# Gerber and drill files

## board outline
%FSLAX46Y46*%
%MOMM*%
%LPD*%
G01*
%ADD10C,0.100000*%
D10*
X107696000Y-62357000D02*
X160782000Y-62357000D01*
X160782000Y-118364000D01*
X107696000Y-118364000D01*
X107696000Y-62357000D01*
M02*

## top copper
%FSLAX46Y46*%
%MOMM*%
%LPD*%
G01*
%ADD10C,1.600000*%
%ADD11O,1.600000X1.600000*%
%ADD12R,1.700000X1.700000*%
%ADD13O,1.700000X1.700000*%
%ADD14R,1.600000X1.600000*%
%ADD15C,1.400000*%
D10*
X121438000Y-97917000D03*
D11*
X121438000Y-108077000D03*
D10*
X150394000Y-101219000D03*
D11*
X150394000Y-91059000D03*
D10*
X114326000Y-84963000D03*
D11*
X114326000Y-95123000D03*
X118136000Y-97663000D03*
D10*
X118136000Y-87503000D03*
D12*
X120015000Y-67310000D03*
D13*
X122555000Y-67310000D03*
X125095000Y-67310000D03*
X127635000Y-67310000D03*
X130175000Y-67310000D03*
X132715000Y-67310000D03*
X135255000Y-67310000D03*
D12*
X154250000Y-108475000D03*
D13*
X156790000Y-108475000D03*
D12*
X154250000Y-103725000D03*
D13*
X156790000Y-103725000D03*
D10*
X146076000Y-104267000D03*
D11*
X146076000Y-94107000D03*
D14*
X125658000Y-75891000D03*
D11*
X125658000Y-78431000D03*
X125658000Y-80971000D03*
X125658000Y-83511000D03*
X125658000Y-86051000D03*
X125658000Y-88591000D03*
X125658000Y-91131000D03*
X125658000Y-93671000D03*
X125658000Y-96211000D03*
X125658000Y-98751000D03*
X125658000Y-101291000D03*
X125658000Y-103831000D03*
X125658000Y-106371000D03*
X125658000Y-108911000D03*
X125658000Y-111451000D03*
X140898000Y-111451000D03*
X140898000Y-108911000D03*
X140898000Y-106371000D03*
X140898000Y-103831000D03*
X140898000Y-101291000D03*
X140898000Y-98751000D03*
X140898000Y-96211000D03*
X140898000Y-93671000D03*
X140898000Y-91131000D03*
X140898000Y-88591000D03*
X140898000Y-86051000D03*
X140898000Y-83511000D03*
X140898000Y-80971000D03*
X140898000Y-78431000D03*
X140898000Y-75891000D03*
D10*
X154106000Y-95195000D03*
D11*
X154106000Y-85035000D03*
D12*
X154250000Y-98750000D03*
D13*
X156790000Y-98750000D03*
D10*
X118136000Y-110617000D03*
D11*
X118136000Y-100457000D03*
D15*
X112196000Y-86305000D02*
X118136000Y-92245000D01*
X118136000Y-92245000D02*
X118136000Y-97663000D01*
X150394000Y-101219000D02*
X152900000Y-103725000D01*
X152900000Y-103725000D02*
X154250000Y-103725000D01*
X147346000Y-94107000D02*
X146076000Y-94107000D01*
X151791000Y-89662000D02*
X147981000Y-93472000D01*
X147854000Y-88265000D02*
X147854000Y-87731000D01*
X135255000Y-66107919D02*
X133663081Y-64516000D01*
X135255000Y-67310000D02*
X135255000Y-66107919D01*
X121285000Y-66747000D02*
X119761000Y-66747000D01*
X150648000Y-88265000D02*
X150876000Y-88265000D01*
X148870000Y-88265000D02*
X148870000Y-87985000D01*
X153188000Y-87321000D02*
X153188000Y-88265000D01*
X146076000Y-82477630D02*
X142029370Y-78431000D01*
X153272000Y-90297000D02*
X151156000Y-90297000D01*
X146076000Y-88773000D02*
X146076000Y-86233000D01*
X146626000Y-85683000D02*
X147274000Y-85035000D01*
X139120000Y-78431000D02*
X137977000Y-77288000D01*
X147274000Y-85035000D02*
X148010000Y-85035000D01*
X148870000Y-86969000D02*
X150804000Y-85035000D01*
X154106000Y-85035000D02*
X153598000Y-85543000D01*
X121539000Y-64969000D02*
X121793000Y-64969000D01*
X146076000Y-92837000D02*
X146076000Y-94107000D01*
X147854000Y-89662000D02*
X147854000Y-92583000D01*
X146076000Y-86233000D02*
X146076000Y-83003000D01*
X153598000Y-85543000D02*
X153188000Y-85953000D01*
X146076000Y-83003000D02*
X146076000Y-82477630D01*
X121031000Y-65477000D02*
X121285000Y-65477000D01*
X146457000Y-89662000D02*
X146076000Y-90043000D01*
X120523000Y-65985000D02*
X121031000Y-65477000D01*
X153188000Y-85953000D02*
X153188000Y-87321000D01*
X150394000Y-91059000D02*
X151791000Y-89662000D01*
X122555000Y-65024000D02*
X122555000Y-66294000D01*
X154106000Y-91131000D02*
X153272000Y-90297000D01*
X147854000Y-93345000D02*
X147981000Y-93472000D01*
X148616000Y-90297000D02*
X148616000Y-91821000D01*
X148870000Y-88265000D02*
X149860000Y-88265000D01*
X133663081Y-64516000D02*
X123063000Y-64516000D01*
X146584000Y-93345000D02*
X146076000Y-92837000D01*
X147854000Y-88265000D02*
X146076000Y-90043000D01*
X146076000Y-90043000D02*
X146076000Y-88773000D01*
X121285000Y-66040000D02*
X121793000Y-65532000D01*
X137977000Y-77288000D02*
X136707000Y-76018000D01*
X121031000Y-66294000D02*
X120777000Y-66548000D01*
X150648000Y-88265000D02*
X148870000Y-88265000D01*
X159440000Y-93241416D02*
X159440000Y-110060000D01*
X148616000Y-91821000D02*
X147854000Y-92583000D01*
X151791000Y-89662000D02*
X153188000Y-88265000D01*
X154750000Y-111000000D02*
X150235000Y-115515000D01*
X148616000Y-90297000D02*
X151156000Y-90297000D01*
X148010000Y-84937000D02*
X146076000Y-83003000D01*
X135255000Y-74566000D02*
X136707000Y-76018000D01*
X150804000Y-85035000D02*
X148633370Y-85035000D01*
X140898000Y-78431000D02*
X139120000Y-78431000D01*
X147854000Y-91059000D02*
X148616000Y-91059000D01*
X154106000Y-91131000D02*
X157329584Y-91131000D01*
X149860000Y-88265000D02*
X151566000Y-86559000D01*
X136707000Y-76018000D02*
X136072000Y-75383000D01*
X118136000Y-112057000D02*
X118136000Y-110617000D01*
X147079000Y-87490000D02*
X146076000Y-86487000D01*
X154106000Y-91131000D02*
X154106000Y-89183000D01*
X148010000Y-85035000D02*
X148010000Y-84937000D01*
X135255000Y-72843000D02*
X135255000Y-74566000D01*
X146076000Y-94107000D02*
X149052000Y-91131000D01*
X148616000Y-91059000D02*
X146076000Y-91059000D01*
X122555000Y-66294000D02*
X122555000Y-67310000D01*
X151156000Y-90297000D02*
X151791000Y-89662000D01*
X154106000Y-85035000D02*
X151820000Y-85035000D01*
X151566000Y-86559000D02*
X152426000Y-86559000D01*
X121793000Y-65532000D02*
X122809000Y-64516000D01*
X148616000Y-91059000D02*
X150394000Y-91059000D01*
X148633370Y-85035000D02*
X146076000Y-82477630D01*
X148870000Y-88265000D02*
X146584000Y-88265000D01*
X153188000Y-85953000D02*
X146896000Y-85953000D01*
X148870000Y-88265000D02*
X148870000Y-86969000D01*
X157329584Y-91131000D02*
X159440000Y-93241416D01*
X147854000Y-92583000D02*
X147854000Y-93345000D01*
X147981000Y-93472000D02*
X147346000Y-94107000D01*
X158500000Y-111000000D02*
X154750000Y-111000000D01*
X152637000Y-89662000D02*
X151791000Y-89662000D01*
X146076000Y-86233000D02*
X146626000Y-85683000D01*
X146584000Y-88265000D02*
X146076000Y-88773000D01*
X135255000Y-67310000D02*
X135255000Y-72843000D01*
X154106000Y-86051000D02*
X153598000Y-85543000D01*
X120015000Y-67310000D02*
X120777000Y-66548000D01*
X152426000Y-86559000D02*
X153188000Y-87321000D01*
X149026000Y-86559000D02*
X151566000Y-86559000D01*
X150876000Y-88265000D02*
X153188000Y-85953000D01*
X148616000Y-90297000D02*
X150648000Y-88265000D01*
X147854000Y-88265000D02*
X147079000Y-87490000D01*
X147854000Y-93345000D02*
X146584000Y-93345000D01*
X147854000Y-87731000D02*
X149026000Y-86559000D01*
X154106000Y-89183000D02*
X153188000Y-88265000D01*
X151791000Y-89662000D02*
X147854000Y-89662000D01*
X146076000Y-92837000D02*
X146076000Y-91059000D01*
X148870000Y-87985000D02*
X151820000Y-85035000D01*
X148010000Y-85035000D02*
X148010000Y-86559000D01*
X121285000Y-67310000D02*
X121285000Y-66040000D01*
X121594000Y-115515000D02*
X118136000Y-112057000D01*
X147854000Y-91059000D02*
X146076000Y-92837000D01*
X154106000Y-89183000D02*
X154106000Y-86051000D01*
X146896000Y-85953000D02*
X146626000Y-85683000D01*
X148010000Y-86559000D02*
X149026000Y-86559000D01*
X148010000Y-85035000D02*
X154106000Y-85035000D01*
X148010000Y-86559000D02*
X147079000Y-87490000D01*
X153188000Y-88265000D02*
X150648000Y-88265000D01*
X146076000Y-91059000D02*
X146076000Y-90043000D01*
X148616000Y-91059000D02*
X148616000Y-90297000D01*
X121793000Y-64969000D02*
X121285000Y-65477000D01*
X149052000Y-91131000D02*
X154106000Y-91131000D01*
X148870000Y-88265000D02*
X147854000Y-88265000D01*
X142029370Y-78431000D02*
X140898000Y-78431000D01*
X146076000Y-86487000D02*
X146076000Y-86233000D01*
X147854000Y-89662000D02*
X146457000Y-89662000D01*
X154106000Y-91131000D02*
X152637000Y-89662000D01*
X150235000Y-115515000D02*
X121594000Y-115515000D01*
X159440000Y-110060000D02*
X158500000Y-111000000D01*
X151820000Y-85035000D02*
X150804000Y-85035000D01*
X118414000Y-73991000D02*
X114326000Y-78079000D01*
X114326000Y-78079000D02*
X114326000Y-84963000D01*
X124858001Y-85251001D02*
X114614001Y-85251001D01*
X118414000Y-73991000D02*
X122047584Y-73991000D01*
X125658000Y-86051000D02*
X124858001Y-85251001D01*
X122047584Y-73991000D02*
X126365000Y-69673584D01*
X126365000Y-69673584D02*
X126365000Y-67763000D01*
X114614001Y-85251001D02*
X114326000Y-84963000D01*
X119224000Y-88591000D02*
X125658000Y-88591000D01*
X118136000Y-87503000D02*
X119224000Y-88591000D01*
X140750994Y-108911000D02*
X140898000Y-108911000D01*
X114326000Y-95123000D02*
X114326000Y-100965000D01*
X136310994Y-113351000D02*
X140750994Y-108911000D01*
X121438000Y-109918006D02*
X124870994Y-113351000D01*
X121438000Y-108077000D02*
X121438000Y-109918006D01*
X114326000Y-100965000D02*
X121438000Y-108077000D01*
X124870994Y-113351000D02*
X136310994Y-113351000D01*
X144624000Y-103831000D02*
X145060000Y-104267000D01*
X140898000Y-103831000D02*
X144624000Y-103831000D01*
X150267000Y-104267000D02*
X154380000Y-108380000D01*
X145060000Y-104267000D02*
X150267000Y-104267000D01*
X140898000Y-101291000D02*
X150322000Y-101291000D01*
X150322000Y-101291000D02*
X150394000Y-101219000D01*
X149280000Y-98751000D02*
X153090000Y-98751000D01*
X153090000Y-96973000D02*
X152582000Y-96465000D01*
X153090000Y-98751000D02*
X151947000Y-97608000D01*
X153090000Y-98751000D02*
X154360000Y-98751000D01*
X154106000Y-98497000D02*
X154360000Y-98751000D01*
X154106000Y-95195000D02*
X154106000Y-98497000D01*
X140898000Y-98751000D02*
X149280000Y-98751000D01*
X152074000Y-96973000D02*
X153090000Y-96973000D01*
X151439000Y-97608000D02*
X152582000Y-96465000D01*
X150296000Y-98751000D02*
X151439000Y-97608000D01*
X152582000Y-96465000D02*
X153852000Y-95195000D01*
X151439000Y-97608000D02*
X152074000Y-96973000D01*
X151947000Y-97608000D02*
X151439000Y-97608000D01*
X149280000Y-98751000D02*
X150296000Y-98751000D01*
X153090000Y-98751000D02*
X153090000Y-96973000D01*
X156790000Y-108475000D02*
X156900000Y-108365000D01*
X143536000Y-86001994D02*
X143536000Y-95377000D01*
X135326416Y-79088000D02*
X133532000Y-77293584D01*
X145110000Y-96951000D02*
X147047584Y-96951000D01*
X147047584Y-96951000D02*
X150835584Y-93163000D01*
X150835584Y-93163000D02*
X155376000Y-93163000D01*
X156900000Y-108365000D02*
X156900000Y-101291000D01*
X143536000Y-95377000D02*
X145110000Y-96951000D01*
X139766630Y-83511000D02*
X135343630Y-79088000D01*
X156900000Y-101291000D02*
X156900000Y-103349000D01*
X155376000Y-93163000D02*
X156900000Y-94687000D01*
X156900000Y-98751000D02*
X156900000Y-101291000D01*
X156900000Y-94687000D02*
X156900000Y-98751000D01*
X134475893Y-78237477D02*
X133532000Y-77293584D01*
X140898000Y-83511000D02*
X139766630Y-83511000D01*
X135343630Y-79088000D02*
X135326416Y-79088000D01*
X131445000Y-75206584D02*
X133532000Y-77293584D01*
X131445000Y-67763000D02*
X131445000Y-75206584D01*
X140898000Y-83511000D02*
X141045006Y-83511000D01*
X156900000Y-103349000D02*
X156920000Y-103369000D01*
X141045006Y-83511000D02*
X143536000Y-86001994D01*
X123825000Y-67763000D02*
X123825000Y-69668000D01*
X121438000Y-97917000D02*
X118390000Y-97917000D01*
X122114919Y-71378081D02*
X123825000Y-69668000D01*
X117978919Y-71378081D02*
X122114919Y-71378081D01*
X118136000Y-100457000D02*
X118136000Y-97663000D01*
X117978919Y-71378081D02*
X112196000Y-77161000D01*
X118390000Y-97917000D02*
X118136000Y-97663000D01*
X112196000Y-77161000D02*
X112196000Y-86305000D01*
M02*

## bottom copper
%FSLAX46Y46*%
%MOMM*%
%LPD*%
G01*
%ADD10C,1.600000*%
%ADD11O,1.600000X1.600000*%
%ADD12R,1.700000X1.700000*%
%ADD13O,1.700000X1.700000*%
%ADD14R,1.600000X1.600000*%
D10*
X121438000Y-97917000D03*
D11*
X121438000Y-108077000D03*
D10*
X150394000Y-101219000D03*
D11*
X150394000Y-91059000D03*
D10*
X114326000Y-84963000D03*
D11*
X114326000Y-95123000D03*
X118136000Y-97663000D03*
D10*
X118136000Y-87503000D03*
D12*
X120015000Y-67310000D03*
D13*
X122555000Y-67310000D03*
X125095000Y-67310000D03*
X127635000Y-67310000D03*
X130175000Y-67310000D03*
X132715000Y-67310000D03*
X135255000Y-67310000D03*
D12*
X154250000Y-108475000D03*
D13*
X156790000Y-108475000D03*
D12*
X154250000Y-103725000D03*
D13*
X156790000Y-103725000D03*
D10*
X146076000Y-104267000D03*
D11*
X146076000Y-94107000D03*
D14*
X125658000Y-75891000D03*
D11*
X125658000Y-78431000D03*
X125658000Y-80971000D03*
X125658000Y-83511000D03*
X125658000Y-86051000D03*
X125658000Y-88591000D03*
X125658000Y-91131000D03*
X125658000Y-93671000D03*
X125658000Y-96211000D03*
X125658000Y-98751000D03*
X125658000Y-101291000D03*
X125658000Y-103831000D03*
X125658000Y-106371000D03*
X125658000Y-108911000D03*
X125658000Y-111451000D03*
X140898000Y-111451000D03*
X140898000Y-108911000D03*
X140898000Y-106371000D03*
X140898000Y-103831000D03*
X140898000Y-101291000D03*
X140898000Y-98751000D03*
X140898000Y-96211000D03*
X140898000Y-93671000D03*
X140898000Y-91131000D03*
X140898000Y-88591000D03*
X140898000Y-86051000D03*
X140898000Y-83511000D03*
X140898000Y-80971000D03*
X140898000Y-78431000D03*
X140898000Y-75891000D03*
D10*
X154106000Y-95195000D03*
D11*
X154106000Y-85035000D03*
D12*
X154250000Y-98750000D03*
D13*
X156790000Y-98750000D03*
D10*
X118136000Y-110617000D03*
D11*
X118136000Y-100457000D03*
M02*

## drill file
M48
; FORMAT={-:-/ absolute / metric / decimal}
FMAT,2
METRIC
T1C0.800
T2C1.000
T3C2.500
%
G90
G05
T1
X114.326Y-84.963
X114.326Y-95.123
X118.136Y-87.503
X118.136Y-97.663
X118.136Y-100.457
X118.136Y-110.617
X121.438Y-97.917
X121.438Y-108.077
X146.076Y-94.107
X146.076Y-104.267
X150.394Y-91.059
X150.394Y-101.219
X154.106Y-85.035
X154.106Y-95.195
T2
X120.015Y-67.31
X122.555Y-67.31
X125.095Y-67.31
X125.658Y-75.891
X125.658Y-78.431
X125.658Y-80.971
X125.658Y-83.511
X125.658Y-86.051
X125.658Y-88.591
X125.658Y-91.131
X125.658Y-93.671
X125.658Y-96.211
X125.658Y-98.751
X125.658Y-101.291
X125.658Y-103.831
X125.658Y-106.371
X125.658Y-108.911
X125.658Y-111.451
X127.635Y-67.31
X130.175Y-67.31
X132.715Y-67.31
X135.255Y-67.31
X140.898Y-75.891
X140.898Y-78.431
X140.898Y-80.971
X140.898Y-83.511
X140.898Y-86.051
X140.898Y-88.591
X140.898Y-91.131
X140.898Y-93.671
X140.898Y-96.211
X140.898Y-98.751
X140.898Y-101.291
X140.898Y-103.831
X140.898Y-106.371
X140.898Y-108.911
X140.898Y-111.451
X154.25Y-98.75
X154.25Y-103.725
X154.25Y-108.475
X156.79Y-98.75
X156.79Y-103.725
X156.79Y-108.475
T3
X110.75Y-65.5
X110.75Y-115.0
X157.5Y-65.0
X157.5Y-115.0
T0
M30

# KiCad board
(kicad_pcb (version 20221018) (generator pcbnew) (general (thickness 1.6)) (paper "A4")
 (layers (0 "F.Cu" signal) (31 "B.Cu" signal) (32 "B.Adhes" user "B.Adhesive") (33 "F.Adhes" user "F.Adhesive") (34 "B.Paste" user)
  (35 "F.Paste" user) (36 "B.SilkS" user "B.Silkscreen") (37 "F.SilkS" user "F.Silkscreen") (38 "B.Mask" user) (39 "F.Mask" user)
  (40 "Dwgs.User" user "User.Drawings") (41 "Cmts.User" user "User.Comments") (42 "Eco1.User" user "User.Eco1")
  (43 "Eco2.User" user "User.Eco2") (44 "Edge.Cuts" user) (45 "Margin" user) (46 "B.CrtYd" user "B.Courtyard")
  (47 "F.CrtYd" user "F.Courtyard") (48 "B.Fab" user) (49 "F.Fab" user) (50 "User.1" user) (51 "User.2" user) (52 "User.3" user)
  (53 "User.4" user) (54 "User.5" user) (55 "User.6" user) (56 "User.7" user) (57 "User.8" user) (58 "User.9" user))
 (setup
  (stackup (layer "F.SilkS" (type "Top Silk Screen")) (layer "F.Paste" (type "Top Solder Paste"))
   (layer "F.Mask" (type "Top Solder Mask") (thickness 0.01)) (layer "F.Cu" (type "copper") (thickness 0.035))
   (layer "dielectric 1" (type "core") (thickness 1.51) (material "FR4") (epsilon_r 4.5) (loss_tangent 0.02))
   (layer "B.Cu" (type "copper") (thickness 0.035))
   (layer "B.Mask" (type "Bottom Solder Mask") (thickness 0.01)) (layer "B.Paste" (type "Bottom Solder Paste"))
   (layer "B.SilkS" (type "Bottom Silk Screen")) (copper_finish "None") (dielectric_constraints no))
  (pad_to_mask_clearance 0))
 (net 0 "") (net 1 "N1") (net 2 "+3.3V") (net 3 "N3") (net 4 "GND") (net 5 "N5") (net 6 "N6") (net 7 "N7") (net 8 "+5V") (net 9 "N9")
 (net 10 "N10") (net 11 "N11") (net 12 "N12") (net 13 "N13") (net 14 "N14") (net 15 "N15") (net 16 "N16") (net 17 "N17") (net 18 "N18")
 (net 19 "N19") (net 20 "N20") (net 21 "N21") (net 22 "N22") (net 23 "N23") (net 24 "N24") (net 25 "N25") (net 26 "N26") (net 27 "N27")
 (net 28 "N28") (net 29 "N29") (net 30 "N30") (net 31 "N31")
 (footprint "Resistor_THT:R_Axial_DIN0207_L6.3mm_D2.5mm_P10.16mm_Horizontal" (layer "F.Cu") (at 121.438 97.917 -90)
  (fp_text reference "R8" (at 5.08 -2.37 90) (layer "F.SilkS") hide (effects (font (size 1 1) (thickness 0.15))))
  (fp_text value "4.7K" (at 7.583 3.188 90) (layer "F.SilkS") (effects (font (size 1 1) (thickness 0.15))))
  (pad "1" thru_hole circle (at 0 0 270) (size 1.6 1.6) (drill 0.8) (layers "*.Cu" "*.Mask") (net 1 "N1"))
  (pad "2" thru_hole oval (at 10.16 0 270) (size 1.6 1.6) (drill 0.8) (layers "*.Cu" "*.Mask") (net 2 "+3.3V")))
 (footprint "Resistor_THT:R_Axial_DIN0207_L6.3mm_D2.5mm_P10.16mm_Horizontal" (layer "F.Cu") (at 150.394 101.219 90)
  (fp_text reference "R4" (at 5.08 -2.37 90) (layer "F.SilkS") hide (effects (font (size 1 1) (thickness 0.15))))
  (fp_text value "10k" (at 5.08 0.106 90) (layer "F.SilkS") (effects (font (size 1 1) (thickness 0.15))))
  (pad "1" thru_hole circle (at 0 0 90) (size 1.6 1.6) (drill 0.8) (layers "*.Cu" "*.Mask") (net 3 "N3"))
  (pad "2" thru_hole oval (at 10.16 0 90) (size 1.6 1.6) (drill 0.8) (layers "*.Cu" "*.Mask") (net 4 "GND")))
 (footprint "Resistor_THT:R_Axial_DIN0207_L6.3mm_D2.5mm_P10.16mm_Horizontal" (layer "F.Cu") (at 114.326 84.963 -90)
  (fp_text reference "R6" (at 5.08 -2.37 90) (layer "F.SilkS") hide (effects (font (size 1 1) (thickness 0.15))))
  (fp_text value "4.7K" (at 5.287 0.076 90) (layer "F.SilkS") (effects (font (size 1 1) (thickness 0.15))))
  (pad "1" thru_hole circle (at 0 0 270) (size 1.6 1.6) (drill 0.8) (layers "*.Cu" "*.Mask") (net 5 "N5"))
  (pad "2" thru_hole oval (at 10.16 0 270) (size 1.6 1.6) (drill 0.8) (layers "*.Cu" "*.Mask") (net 2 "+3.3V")))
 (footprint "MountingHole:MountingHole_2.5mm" (layer "F.Cu") (at 157.5 115)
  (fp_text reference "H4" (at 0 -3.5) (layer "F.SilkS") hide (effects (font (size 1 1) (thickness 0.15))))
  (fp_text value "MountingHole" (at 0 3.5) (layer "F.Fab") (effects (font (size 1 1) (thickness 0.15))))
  (pad "" np_thru_hole circle (at 0 0) (size 2.5 2.5) (drill 2.5) (layers "*.Cu" "*.Mask")))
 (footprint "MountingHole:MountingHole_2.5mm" (layer "F.Cu") (at 110.75 115)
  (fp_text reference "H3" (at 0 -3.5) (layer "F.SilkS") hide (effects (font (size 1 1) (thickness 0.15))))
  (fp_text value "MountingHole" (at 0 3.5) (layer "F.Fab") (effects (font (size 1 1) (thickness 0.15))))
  (pad "" np_thru_hole circle (at 0 0) (size 2.5 2.5) (drill 2.5) (layers "*.Cu" "*.Mask")))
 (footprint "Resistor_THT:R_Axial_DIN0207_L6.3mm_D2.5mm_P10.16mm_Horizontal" (layer "F.Cu") (at 118.136 87.503 -90)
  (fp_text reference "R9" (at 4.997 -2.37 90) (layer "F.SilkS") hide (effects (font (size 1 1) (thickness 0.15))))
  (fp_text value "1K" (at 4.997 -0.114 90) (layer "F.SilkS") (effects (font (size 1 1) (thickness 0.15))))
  (pad "1" thru_hole circle (at 0 0 270) (size 1.6 1.6) (drill 0.8) (layers "*.Cu" "*.Mask") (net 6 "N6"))
  (pad "2" thru_hole oval (at 10.16 0 270) (size 1.6 1.6) (drill 0.8) (layers "*.Cu" "*.Mask") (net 1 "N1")))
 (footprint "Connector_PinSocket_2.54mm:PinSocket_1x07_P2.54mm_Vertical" (layer "F.Cu") (at 120.015 67.31 90)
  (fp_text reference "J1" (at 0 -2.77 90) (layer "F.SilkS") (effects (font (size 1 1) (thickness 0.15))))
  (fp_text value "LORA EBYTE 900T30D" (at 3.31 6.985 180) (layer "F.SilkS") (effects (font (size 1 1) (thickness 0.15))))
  (pad "1" thru_hole rect (at 0 0 90) (size 1.7 1.7) (drill 1) (layers "*.Cu" "*.Mask") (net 4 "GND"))
  (pad "2" thru_hole oval (at 0 2.54 90) (size 1.7 1.7) (drill 1) (layers "*.Cu" "*.Mask") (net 4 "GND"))
  (pad "3" thru_hole oval (at 0 5.08 90) (size 1.7 1.7) (drill 1) (layers "*.Cu" "*.Mask") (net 1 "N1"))
  (pad "4" thru_hole oval (at 0 7.62 90) (size 1.7 1.7) (drill 1) (layers "*.Cu" "*.Mask") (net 5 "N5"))
  (pad "5" thru_hole oval (at 0 10.16 90) (size 1.7 1.7) (drill 1) (layers "*.Cu" "*.Mask") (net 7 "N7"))
  (pad "6" thru_hole oval (at 0 12.7 90) (size 1.7 1.7) (drill 1) (layers "*.Cu" "*.Mask") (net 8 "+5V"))
  (pad "7" thru_hole oval (at 0 15.24 90) (size 1.7 1.7) (drill 1) (layers "*.Cu" "*.Mask") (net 4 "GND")))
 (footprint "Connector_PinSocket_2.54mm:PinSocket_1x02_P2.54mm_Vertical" (layer "F.Cu") (at 154.25 108.475 90)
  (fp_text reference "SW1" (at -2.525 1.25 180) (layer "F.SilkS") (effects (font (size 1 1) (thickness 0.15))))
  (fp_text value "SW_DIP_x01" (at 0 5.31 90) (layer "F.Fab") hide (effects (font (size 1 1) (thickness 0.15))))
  (pad "1" thru_hole rect (at 0 0 90) (size 1.7 1.7) (drill 1) (layers "*.Cu" "*.Mask") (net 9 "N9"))
  (pad "2" thru_hole oval (at 0 2.54 90) (size 1.7 1.7) (drill 1) (layers "*.Cu" "*.Mask") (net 8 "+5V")))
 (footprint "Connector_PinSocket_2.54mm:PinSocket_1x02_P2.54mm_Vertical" (layer "F.Cu") (at 154.25 103.725 90)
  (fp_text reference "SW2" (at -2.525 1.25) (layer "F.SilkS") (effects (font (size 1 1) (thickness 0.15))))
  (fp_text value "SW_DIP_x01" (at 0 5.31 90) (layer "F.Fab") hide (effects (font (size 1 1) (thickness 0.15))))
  (pad "1" thru_hole rect (at 0 0 90) (size 1.7 1.7) (drill 1) (layers "*.Cu" "*.Mask") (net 3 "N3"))
  (pad "2" thru_hole oval (at 0 2.54 90) (size 1.7 1.7) (drill 1) (layers "*.Cu" "*.Mask") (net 8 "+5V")))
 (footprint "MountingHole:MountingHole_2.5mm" (layer "F.Cu") (at 110.75 65.5)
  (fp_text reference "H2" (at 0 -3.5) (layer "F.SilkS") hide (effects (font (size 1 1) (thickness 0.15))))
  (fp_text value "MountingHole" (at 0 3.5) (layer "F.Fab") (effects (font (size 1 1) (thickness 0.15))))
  (pad "" np_thru_hole circle (at 0 0) (size 2.5 2.5) (drill 2.5) (layers "*.Cu" "*.Mask")))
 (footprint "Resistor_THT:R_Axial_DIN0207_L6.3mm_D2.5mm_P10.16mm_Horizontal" (layer "F.Cu") (at 146.076 104.267 90)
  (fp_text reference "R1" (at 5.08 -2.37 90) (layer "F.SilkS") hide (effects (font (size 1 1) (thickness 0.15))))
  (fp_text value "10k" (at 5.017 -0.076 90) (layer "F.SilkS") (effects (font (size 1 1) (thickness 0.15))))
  (pad "1" thru_hole circle (at 0 0 90) (size 1.6 1.6) (drill 0.8) (layers "*.Cu" "*.Mask") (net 9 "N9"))
  (pad "2" thru_hole oval (at 10.16 0 90) (size 1.6 1.6) (drill 0.8) (layers "*.Cu" "*.Mask") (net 4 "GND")))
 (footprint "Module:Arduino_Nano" (layer "F.Cu") (at 125.658 75.891)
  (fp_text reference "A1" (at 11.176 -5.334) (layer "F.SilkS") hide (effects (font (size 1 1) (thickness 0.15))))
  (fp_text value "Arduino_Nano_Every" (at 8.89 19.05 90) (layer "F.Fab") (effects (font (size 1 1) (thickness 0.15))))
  (pad "1" thru_hole rect (at 0 0) (size 1.6 1.6) (drill 1) (layers "*.Cu" "*.Mask") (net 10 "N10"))
  (pad "2" thru_hole oval (at 0 2.54) (size 1.6 1.6) (drill 1) (layers "*.Cu" "*.Mask") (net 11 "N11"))
  (pad "3" thru_hole oval (at 0 5.08) (size 1.6 1.6) (drill 1) (layers "*.Cu" "*.Mask") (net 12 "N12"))
  (pad "4" thru_hole oval (at 0 7.62) (size 1.6 1.6) (drill 1) (layers "*.Cu" "*.Mask") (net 4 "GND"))
  (pad "5" thru_hole oval (at 0 10.16) (size 1.6 1.6) (drill 1) (layers "*.Cu" "*.Mask") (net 5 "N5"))
  (pad "6" thru_hole oval (at 0 12.7) (size 1.6 1.6) (drill 1) (layers "*.Cu" "*.Mask") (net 6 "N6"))
  (pad "7" thru_hole oval (at 0 15.24) (size 1.6 1.6) (drill 1) (layers "*.Cu" "*.Mask") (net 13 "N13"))
  (pad "8" thru_hole oval (at 0 17.78) (size 1.6 1.6) (drill 1) (layers "*.Cu" "*.Mask") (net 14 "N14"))
  (pad "9" thru_hole oval (at 0 20.32) (size 1.6 1.6) (drill 1) (layers "*.Cu" "*.Mask") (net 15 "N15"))
  (pad "10" thru_hole oval (at 0 22.86) (size 1.6 1.6) (drill 1) (layers "*.Cu" "*.Mask") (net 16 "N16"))
  (pad "11" thru_hole oval (at 0 25.4) (size 1.6 1.6) (drill 1) (layers "*.Cu" "*.Mask") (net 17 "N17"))
  (pad "12" thru_hole oval (at 0 27.94) (size 1.6 1.6) (drill 1) (layers "*.Cu" "*.Mask") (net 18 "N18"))
  (pad "13" thru_hole oval (at 0 30.48) (size 1.6 1.6) (drill 1) (layers "*.Cu" "*.Mask") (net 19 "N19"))
  (pad "14" thru_hole oval (at 0 33.02) (size 1.6 1.6) (drill 1) (layers "*.Cu" "*.Mask") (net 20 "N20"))
  (pad "15" thru_hole oval (at 0 35.56) (size 1.6 1.6) (drill 1) (layers "*.Cu" "*.Mask") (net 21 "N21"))
  (pad "16" thru_hole oval (at 15.24 35.56) (size 1.6 1.6) (drill 1) (layers "*.Cu" "*.Mask") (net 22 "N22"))
  (pad "17" thru_hole oval (at 15.24 33.02) (size 1.6 1.6) (drill 1) (layers "*.Cu" "*.Mask") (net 2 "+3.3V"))
  (pad "18" thru_hole oval (at 15.24 30.48) (size 1.6 1.6) (drill 1) (layers "*.Cu" "*.Mask") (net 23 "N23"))
  (pad "19" thru_hole oval (at 15.24 27.94) (size 1.6 1.6) (drill 1) (layers "*.Cu" "*.Mask") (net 9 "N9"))
  (pad "20" thru_hole oval (at 15.24 25.4) (size 1.6 1.6) (drill 1) (layers "*.Cu" "*.Mask") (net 3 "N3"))
  (pad "21" thru_hole oval (at 15.24 22.86) (size 1.6 1.6) (drill 1) (layers "*.Cu" "*.Mask") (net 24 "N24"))
  (pad "22" thru_hole oval (at 15.24 20.32) (size 1.6 1.6) (drill 1) (layers "*.Cu" "*.Mask") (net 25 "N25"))
  (pad "23" thru_hole oval (at 15.24 17.78) (size 1.6 1.6) (drill 1) (layers "*.Cu" "*.Mask") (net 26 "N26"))
  (pad "24" thru_hole oval (at 15.24 15.24) (size 1.6 1.6) (drill 1) (layers "*.Cu" "*.Mask") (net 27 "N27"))
  (pad "25" thru_hole oval (at 15.24 12.7) (size 1.6 1.6) (drill 1) (layers "*.Cu" "*.Mask") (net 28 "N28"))
  (pad "26" thru_hole oval (at 15.24 10.16) (size 1.6 1.6) (drill 1) (layers "*.Cu" "*.Mask") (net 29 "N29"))
  (pad "27" thru_hole oval (at 15.24 7.62) (size 1.6 1.6) (drill 1) (layers "*.Cu" "*.Mask") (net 8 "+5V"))
  (pad "28" thru_hole oval (at 15.24 5.08) (size 1.6 1.6) (drill 1) (layers "*.Cu" "*.Mask") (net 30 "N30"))
  (pad "29" thru_hole oval (at 15.24 2.54) (size 1.6 1.6) (drill 1) (layers "*.Cu" "*.Mask") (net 4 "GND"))
  (pad "30" thru_hole oval (at 15.24 0) (size 1.6 1.6) (drill 1) (layers "*.Cu" "*.Mask") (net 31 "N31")))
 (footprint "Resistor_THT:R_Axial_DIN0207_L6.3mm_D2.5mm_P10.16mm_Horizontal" (layer "F.Cu") (at 154.106 95.195 90)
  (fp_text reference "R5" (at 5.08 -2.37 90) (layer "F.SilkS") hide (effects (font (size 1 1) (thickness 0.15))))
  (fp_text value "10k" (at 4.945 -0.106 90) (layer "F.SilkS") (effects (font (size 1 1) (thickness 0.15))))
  (pad "1" thru_hole circle (at 0 0 90) (size 1.6 1.6) (drill 0.8) (layers "*.Cu" "*.Mask") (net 24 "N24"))
  (pad "2" thru_hole oval (at 10.16 0 90) (size 1.6 1.6) (drill 0.8) (layers "*.Cu" "*.Mask") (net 4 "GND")))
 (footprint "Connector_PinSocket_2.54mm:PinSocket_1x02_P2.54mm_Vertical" (layer "F.Cu") (at 154.25 98.75 90)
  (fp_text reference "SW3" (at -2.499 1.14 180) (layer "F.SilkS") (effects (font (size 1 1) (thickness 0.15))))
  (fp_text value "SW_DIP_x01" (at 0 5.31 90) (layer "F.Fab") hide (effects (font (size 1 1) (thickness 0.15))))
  (pad "1" thru_hole rect (at 0 0 90) (size 1.7 1.7) (drill 1) (layers "*.Cu" "*.Mask") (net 24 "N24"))
  (pad "2" thru_hole oval (at 0 2.54 90) (size 1.7 1.7) (drill 1) (layers "*.Cu" "*.Mask") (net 8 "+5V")))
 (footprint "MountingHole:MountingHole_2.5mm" (layer "F.Cu") (at 157.5 65)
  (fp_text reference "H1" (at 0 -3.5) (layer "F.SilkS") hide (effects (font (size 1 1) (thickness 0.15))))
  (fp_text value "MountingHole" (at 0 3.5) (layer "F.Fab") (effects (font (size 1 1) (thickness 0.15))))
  (pad "" np_thru_hole circle (at 0 0) (size 2.5 2.5) (drill 2.5) (layers "*.Cu" "*.Mask")))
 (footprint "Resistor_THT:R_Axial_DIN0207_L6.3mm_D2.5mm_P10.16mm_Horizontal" (layer "F.Cu") (at 118.136 110.617 90)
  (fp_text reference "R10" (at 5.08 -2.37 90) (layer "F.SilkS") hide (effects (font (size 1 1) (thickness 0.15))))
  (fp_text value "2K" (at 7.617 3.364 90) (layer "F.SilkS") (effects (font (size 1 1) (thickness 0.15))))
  (pad "1" thru_hole circle (at 0 0 90) (size 1.6 1.6) (drill 0.8) (layers "*.Cu" "*.Mask") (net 4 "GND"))
  (pad "2" thru_hole oval (at 10.16 0 90) (size 1.6 1.6) (drill 0.8) (layers "*.Cu" "*.Mask") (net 1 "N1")))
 (gr_rect (start 107.696 62.357) (end 160.782 118.364) (stroke (width 0.1) (type default)) (fill none) (layer "Edge.Cuts"))
 (segment (start 147.346 94.107) (end 146.076 94.107) (width 1.4) (layer "F.Cu") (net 4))
 (segment (start 151.791 89.662) (end 147.981 93.472) (width 1.4) (layer "F.Cu") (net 4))
 (segment (start 147.854 88.265) (end 147.854 87.731) (width 1.4) (layer "F.Cu") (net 4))
 (segment (start 135.255 66.107919) (end 133.663081 64.516) (width 1.4) (layer "F.Cu") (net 4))
 (segment (start 135.255 67.31) (end 135.255 66.107919) (width 1.4) (layer "F.Cu") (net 4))
 (segment (start 121.285 66.747) (end 119.761 66.747) (width 1.4) (layer "F.Cu") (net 4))
 (segment (start 150.648 88.265) (end 150.876 88.265) (width 1.4) (layer "F.Cu") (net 4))
 (segment (start 148.87 88.265) (end 148.87 87.985) (width 1.4) (layer "F.Cu") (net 4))
 (segment (start 153.188 87.321) (end 153.188 88.265) (width 1.4) (layer "F.Cu") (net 4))
 (segment (start 146.076 82.47763) (end 142.02937 78.431) (width 1.4) (layer "F.Cu") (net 4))
 (segment (start 153.272 90.297) (end 151.156 90.297) (width 1.4) (layer "F.Cu") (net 4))
 (segment (start 146.076 88.773) (end 146.076 86.233) (width 1.4) (layer "F.Cu") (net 4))
 (segment (start 146.626 85.683) (end 147.274 85.035) (width 1.4) (layer "F.Cu") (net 4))
 (segment (start 139.12 78.431) (end 137.977 77.288) (width 1.4) (layer "F.Cu") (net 4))
 (segment (start 147.274 85.035) (end 148.01 85.035) (width 1.4) (layer "F.Cu") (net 4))
 (segment (start 148.87 86.969) (end 150.804 85.035) (width 1.4) (layer "F.Cu") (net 4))
 (segment (start 154.106 85.035) (end 153.598 85.543) (width 1.4) (layer "F.Cu") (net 4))
 (segment (start 121.539 64.969) (end 121.793 64.969) (width 1.4) (layer "F.Cu") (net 4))
 (segment (start 146.076 92.837) (end 146.076 94.107) (width 1.4) (layer "F.Cu") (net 4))
 (segment (start 147.854 89.662) (end 147.854 92.583) (width 1.4) (layer "F.Cu") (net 4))
 (segment (start 146.076 86.233) (end 146.076 83.003) (width 1.4) (layer "F.Cu") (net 4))
 (segment (start 153.598 85.543) (end 153.188 85.953) (width 1.4) (layer "F.Cu") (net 4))
 (segment (start 146.076 83.003) (end 146.076 82.47763) (width 1.4) (layer "F.Cu") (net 4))
 (segment (start 121.031 65.477) (end 121.285 65.477) (width 1.4) (layer "F.Cu") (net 4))
 (segment (start 146.457 89.662) (end 146.076 90.043) (width 1.4) (layer "F.Cu") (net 4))
 (segment (start 120.523 65.985) (end 121.031 65.477) (width 1.4) (layer "F.Cu") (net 4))
 (segment (start 153.188 85.953) (end 153.188 87.321) (width 1.4) (layer "F.Cu") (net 4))
 (segment (start 150.394 91.059) (end 151.791 89.662) (width 1.4) (layer "F.Cu") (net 4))
 (segment (start 122.555 65.024) (end 122.555 66.294) (width 1.4) (layer "F.Cu") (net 4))
 (segment (start 154.106 91.131) (end 153.272 90.297) (width 1.4) (layer "F.Cu") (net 4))
 (segment (start 147.854 93.345) (end 147.981 93.472) (width 1.4) (layer "F.Cu") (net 4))
 (segment (start 148.616 90.297) (end 148.616 91.821) (width 1.4) (layer "F.Cu") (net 4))
 (segment (start 148.87 88.265) (end 149.86 88.265) (width 1.4) (layer "F.Cu") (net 4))
 (segment (start 133.663081 64.516) (end 123.063 64.516) (width 1.4) (layer "F.Cu") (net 4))
 (segment (start 146.584 93.345) (end 146.076 92.837) (width 1.4) (layer "F.Cu") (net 4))
 (segment (start 147.854 88.265) (end 146.076 90.043) (width 1.4) (layer "F.Cu") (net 4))
 (segment (start 146.076 90.043) (end 146.076 88.773) (width 1.4) (layer "F.Cu") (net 4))
 (segment (start 121.285 66.04) (end 121.793 65.532) (width 1.4) (layer "F.Cu") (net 4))
 (segment (start 137.977 77.288) (end 136.707 76.018) (width 1.4) (layer "F.Cu") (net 4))
 (segment (start 121.031 66.294) (end 120.777 66.548) (width 1.4) (layer "F.Cu") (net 4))
 (segment (start 150.648 88.265) (end 148.87 88.265) (width 1.4) (layer "F.Cu") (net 4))
 (segment (start 159.44 93.241416) (end 159.44 110.06) (width 1.4) (layer "F.Cu") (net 4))
 (segment (start 148.616 91.821) (end 147.854 92.583) (width 1.4) (layer "F.Cu") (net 4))
 (segment (start 151.791 89.662) (end 153.188 88.265) (width 1.4) (layer "F.Cu") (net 4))
 (segment (start 154.75 111) (end 150.235 115.515) (width 1.4) (layer "F.Cu") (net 4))
 (segment (start 148.616 90.297) (end 151.156 90.297) (width 1.4) (layer "F.Cu") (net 4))
 (segment (start 148.01 84.937) (end 146.076 83.003) (width 1.4) (layer "F.Cu") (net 4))
 (segment (start 135.255 74.566) (end 136.707 76.018) (width 1.4) (layer "F.Cu") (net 4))
 (segment (start 150.804 85.035) (end 148.63337 85.035) (width 1.4) (layer "F.Cu") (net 4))
 (segment (start 140.898 78.431) (end 139.12 78.431) (width 1.4) (layer "F.Cu") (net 4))
 (segment (start 147.854 91.059) (end 148.616 91.059) (width 1.4) (layer "F.Cu") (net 4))
 (segment (start 154.106 91.131) (end 157.329584 91.131) (width 1.4) (layer "F.Cu") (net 4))
 (segment (start 149.86 88.265) (end 151.566 86.559) (width 1.4) (layer "F.Cu") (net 4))
 (segment (start 136.707 76.018) (end 136.072 75.383) (width 1.4) (layer "F.Cu") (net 4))
 (segment (start 118.136 112.057) (end 118.136 110.617) (width 1.4) (layer "F.Cu") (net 4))
 (segment (start 147.079 87.49) (end 146.076 86.487) (width 1.4) (layer "F.Cu") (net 4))
 (segment (start 154.106 91.131) (end 154.106 89.183) (width 1.4) (layer "F.Cu") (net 4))
 (segment (start 148.01 85.035) (end 148.01 84.937) (width 1.4) (layer "F.Cu") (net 4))
 (segment (start 135.255 72.843) (end 135.255 74.566) (width 1.4) (layer "F.Cu") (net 4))
 (segment (start 146.076 94.107) (end 149.052 91.131) (width 1.4) (layer "F.Cu") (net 4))
 (segment (start 148.616 91.059) (end 146.076 91.059) (width 1.4) (layer "F.Cu") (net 4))
 (segment (start 122.555 66.294) (end 122.555 67.31) (width 1.4) (layer "F.Cu") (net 4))
 (segment (start 151.156 90.297) (end 151.791 89.662) (width 1.4) (layer "F.Cu") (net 4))
 (segment (start 154.106 85.035) (end 151.82 85.035) (width 1.4) (layer "F.Cu") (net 4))
 (segment (start 151.566 86.559) (end 152.426 86.559) (width 1.4) (layer "F.Cu") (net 4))
 (segment (start 121.793 65.532) (end 122.809 64.516) (width 1.4) (layer "F.Cu") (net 4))
 (segment (start 148.616 91.059) (end 150.394 91.059) (width 1.4) (layer "F.Cu") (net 4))
 (segment (start 148.63337 85.035) (end 146.076 82.47763) (width 1.4) (layer "F.Cu") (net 4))
 (segment (start 148.87 88.265) (end 146.584 88.265) (width 1.4) (layer "F.Cu") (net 4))
 (segment (start 153.188 85.953) (end 146.896 85.953) (width 1.4) (layer "F.Cu") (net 4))
 (segment (start 148.87 88.265) (end 148.87 86.969) (width 1.4) (layer "F.Cu") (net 4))
 (segment (start 157.329584 91.131) (end 159.44 93.241416) (width 1.4) (layer "F.Cu") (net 4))
 (segment (start 147.854 92.583) (end 147.854 93.345) (width 1.4) (layer "F.Cu") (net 4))
 (segment (start 147.981 93.472) (end 147.346 94.107) (width 1.4) (layer "F.Cu") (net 4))
 (segment (start 158.5 111) (end 154.75 111) (width 1.4) (layer "F.Cu") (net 4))
 (segment (start 152.637 89.662) (end 151.791 89.662) (width 1.4) (layer "F.Cu") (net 4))
 (segment (start 146.076 86.233) (end 146.626 85.683) (width 1.4) (layer "F.Cu") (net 4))
 (segment (start 146.584 88.265) (end 146.076 88.773) (width 1.4) (layer "F.Cu") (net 4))
 (segment (start 135.255 67.31) (end 135.255 72.843) (width 1.4) (layer "F.Cu") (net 4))
 (segment (start 154.106 86.051) (end 153.598 85.543) (width 1.4) (layer "F.Cu") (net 4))
 (segment (start 120.015 67.31) (end 120.777 66.548) (width 1.4) (layer "F.Cu") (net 4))
 (segment (start 152.426 86.559) (end 153.188 87.321) (width 1.4) (layer "F.Cu") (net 4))
 (segment (start 149.026 86.559) (end 151.566 86.559) (width 1.4) (layer "F.Cu") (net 4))
 (segment (start 150.876 88.265) (end 153.188 85.953) (width 1.4) (layer "F.Cu") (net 4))
 (segment (start 148.616 90.297) (end 150.648 88.265) (width 1.4) (layer "F.Cu") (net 4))
 (segment (start 147.854 88.265) (end 147.079 87.49) (width 1.4) (layer "F.Cu") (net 4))
 (segment (start 147.854 93.345) (end 146.584 93.345) (width 1.4) (layer "F.Cu") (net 4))
 (segment (start 147.854 87.731) (end 149.026 86.559) (width 1.4) (layer "F.Cu") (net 4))
 (segment (start 154.106 89.183) (end 153.188 88.265) (width 1.4) (layer "F.Cu") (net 4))
 (segment (start 151.791 89.662) (end 147.854 89.662) (width 1.4) (layer "F.Cu") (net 4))
 (segment (start 146.076 92.837) (end 146.076 91.059) (width 1.4) (layer "F.Cu") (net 4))
 (segment (start 148.87 87.985) (end 151.82 85.035) (width 1.4) (layer "F.Cu") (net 4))
 (segment (start 148.01 85.035) (end 148.01 86.559) (width 1.4) (layer "F.Cu") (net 4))
 (segment (start 121.285 67.31) (end 121.285 66.04) (width 1.4) (layer "F.Cu") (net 4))
 (segment (start 121.594 115.515) (end 118.136 112.057) (width 1.4) (layer "F.Cu") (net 4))
 (segment (start 147.854 91.059) (end 146.076 92.837) (width 1.4) (layer "F.Cu") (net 4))
 (segment (start 154.106 89.183) (end 154.106 86.051) (width 1.4) (layer "F.Cu") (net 4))
 (segment (start 146.896 85.953) (end 146.626 85.683) (width 1.4) (layer "F.Cu") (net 4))
 (segment (start 148.01 86.559) (end 149.026 86.559) (width 1.4) (layer "F.Cu") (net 4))
 (segment (start 148.01 85.035) (end 154.106 85.035) (width 1.4) (layer "F.Cu") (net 4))
 (segment (start 148.01 86.559) (end 147.079 87.49) (width 1.4) (layer "F.Cu") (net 4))
 (segment (start 153.188 88.265) (end 150.648 88.265) (width 1.4) (layer "F.Cu") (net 4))
 (segment (start 146.076 91.059) (end 146.076 90.043) (width 1.4) (layer "F.Cu") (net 4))
 (segment (start 148.616 91.059) (end 148.616 90.297) (width 1.4) (layer "F.Cu") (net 4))
 (segment (start 121.793 64.969) (end 121.285 65.477) (width 1.4) (layer "F.Cu") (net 4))
 (segment (start 149.052 91.131) (end 154.106 91.131) (width 1.4) (layer "F.Cu") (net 4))
 (segment (start 148.87 88.265) (end 147.854 88.265) (width 1.4) (layer "F.Cu") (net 4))
 (segment (start 142.02937 78.431) (end 140.898 78.431) (width 1.4) (layer "F.Cu") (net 4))
 (segment (start 146.076 86.487) (end 146.076 86.233) (width 1.4) (layer "F.Cu") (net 4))
 (segment (start 147.854 89.662) (end 146.457 89.662) (width 1.4) (layer "F.Cu") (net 4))
 (segment (start 154.106 91.131) (end 152.637 89.662) (width 1.4) (layer "F.Cu") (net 4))
 (segment (start 150.235 115.515) (end 121.594 115.515) (width 1.4) (layer "F.Cu") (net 4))
 (segment (start 159.44 110.06) (end 158.5 111) (width 1.4) (layer "F.Cu") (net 4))
 (segment (start 151.82 85.035) (end 150.804 85.035) (width 1.4) (layer "F.Cu") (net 4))
 (segment (start 118.414 73.991) (end 114.326 78.079) (width 1.4) (layer "F.Cu") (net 5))
 (segment (start 114.326 78.079) (end 114.326 84.963) (width 1.4) (layer "F.Cu") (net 5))
 (segment (start 124.858001 85.251001) (end 114.614001 85.251001) (width 1.4) (layer "F.Cu") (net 5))
 (segment (start 118.414 73.991) (end 122.047584 73.991) (width 1.4) (layer "F.Cu") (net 5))
 (segment (start 125.658 86.051) (end 124.858001 85.251001) (width 1.4) (layer "F.Cu") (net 5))
 (segment (start 122.047584 73.991) (end 126.365 69.673584) (width 1.4) (layer "F.Cu") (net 5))
 (segment (start 126.365 69.673584) (end 126.365 67.763) (width 1.4) (layer "F.Cu") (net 5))
 (segment (start 114.614001 85.251001) (end 114.326 84.963) (width 1.4) (layer "F.Cu") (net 5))
 (segment (start 119.224 88.591) (end 125.658 88.591) (width 1.4) (layer "F.Cu") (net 6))
 (segment (start 118.136 87.503) (end 119.224 88.591) (width 1.4) (layer "F.Cu") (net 6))
 (segment (start 140.750994 108.911) (end 140.898 108.911) (width 1.4) (layer "F.Cu") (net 2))
 (segment (start 114.326 95.123) (end 114.326 100.965) (width 1.4) (layer "F.Cu") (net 2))
 (segment (start 136.310994 113.351) (end 140.750994 108.911) (width 1.4) (layer "F.Cu") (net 2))
 (segment (start 121.438 109.918006) (end 124.870994 113.351) (width 1.4) (layer "F.Cu") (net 2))
 (segment (start 121.438 108.077) (end 121.438 109.918006) (width 1.4) (layer "F.Cu") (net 2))
 (segment (start 114.326 100.965) (end 121.438 108.077) (width 1.4) (layer "F.Cu") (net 2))
 (segment (start 124.870994 113.351) (end 136.310994 113.351) (width 1.4) (layer "F.Cu") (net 2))
 (segment (start 144.624 103.831) (end 145.06 104.267) (width 1.4) (layer "F.Cu") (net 9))
 (segment (start 140.898 103.831) (end 144.624 103.831) (width 1.4) (layer "F.Cu") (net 9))
 (segment (start 150.267 104.267) (end 154.38 108.38) (width 1.4) (layer "F.Cu") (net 9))
 (segment (start 145.06 104.267) (end 150.267 104.267) (width 1.4) (layer "F.Cu") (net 9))
 (segment (start 150.394 101.219) (end 152.9 103.725) (width 1.4) (layer "F.Cu") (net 3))
 (segment (start 140.898 101.291) (end 150.322 101.291) (width 1.4) (layer "F.Cu") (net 3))
 (segment (start 150.322 101.291) (end 150.394 101.219) (width 1.4) (layer "F.Cu") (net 3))
 (segment (start 152.9 103.725) (end 154.25 103.725) (width 1.4) (layer "F.Cu") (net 3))
 (segment (start 149.28 98.751) (end 153.09 98.751) (width 1.4) (layer "F.Cu") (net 24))
 (segment (start 153.09 96.973) (end 152.582 96.465) (width 1.4) (layer "F.Cu") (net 24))
 (segment (start 153.09 98.751) (end 151.947 97.608) (width 1.4) (layer "F.Cu") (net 24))
 (segment (start 153.09 98.751) (end 154.36 98.751) (width 1.4) (layer "F.Cu") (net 24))
 (segment (start 154.106 98.497) (end 154.36 98.751) (width 1.4) (layer "F.Cu") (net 24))
 (segment (start 154.106 95.195) (end 154.106 98.497) (width 1.4) (layer "F.Cu") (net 24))
 (segment (start 140.898 98.751) (end 149.28 98.751) (width 1.4) (layer "F.Cu") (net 24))
 (segment (start 152.074 96.973) (end 153.09 96.973) (width 1.4) (layer "F.Cu") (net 24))
 (segment (start 151.439 97.608) (end 152.582 96.465) (width 1.4) (layer "F.Cu") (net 24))
 (segment (start 150.296 98.751) (end 151.439 97.608) (width 1.4) (layer "F.Cu") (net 24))
 (segment (start 152.582 96.465) (end 153.852 95.195) (width 1.4) (layer "F.Cu") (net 24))
 (segment (start 151.439 97.608) (end 152.074 96.973) (width 1.4) (layer "F.Cu") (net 24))
 (segment (start 151.947 97.608) (end 151.439 97.608) (width 1.4) (layer "F.Cu") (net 24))
 (segment (start 149.28 98.751) (end 150.296 98.751) (width 1.4) (layer "F.Cu") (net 24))
 (segment (start 153.09 98.751) (end 153.09 96.973) (width 1.4) (layer "F.Cu") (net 24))
 (segment (start 156.79 108.475) (end 156.9 108.365) (width 1.4) (layer "F.Cu") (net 8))
 (segment (start 143.536 86.001994) (end 143.536 95.377) (width 1.4) (layer "F.Cu") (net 8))
 (segment (start 135.326416 79.088) (end 133.532 77.293584) (width 1.4) (layer "F.Cu") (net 8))
 (segment (start 145.11 96.951) (end 147.047584 96.951) (width 1.4) (layer "F.Cu") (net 8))
 (segment (start 147.047584 96.951) (end 150.835584 93.163) (width 1.4) (layer "F.Cu") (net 8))
 (segment (start 150.835584 93.163) (end 155.376 93.163) (width 1.4) (layer "F.Cu") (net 8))
 (segment (start 156.9 108.365) (end 156.9 101.291) (width 1.4) (layer "F.Cu") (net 8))
 (segment (start 143.536 95.377) (end 145.11 96.951) (width 1.4) (layer "F.Cu") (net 8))
 (segment (start 139.76663 83.511) (end 135.34363 79.088) (width 1.4) (layer "F.Cu") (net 8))
 (segment (start 156.9 101.291) (end 156.9 103.349) (width 1.4) (layer "F.Cu") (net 8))
 (segment (start 155.376 93.163) (end 156.9 94.687) (width 1.4) (layer "F.Cu") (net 8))
 (segment (start 156.9 98.751) (end 156.9 101.291) (width 1.4) (layer "F.Cu") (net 8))
 (segment (start 156.9 94.687) (end 156.9 98.751) (width 1.4) (layer "F.Cu") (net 8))
 (segment (start 134.475893 78.237477) (end 133.532 77.293584) (width 1.4) (layer "F.Cu") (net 8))
 (segment (start 140.898 83.511) (end 139.76663 83.511) (width 1.4) (layer "F.Cu") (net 8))
 (segment (start 135.34363 79.088) (end 135.326416 79.088) (width 1.4) (layer "F.Cu") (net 8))
 (segment (start 131.445 75.206584) (end 133.532 77.293584) (width 1.4) (layer "F.Cu") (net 8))
 (segment (start 131.445 67.763) (end 131.445 75.206584) (width 1.4) (layer "F.Cu") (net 8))
 (segment (start 140.898 83.511) (end 141.045006 83.511) (width 1.4) (layer "F.Cu") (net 8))
 (segment (start 156.9 103.349) (end 156.92 103.369) (width 1.4) (layer "F.Cu") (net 8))
 (segment (start 141.045006 83.511) (end 143.536 86.001994) (width 1.4) (layer "F.Cu") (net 8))
 (segment (start 123.825 67.763) (end 123.825 69.668) (width 1.4) (layer "F.Cu") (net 1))
 (segment (start 121.438 97.917) (end 118.39 97.917) (width 1.4) (layer "F.Cu") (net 1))
 (segment (start 122.114919 71.378081) (end 123.825 69.668) (width 1.4) (layer "F.Cu") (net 1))
 (segment (start 112.196 86.305) (end 118.136 92.245) (width 1.4) (layer "F.Cu") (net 1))
 (segment (start 117.978919 71.378081) (end 122.114919 71.378081) (width 1.4) (layer "F.Cu") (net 1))
 (segment (start 118.136 100.457) (end 118.136 97.663) (width 1.4) (layer "F.Cu") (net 1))
 (segment (start 118.136 92.245) (end 118.136 97.663) (width 1.4) (layer "F.Cu") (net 1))
 (segment (start 117.978919 71.378081) (end 112.196 77.161) (width 1.4) (layer "F.Cu") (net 1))
 (segment (start 118.39 97.917) (end 118.136 97.663) (width 1.4) (layer "F.Cu") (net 1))
 (segment (start 112.196 77.161) (end 112.196 86.305) (width 1.4) (layer "F.Cu") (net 1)))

